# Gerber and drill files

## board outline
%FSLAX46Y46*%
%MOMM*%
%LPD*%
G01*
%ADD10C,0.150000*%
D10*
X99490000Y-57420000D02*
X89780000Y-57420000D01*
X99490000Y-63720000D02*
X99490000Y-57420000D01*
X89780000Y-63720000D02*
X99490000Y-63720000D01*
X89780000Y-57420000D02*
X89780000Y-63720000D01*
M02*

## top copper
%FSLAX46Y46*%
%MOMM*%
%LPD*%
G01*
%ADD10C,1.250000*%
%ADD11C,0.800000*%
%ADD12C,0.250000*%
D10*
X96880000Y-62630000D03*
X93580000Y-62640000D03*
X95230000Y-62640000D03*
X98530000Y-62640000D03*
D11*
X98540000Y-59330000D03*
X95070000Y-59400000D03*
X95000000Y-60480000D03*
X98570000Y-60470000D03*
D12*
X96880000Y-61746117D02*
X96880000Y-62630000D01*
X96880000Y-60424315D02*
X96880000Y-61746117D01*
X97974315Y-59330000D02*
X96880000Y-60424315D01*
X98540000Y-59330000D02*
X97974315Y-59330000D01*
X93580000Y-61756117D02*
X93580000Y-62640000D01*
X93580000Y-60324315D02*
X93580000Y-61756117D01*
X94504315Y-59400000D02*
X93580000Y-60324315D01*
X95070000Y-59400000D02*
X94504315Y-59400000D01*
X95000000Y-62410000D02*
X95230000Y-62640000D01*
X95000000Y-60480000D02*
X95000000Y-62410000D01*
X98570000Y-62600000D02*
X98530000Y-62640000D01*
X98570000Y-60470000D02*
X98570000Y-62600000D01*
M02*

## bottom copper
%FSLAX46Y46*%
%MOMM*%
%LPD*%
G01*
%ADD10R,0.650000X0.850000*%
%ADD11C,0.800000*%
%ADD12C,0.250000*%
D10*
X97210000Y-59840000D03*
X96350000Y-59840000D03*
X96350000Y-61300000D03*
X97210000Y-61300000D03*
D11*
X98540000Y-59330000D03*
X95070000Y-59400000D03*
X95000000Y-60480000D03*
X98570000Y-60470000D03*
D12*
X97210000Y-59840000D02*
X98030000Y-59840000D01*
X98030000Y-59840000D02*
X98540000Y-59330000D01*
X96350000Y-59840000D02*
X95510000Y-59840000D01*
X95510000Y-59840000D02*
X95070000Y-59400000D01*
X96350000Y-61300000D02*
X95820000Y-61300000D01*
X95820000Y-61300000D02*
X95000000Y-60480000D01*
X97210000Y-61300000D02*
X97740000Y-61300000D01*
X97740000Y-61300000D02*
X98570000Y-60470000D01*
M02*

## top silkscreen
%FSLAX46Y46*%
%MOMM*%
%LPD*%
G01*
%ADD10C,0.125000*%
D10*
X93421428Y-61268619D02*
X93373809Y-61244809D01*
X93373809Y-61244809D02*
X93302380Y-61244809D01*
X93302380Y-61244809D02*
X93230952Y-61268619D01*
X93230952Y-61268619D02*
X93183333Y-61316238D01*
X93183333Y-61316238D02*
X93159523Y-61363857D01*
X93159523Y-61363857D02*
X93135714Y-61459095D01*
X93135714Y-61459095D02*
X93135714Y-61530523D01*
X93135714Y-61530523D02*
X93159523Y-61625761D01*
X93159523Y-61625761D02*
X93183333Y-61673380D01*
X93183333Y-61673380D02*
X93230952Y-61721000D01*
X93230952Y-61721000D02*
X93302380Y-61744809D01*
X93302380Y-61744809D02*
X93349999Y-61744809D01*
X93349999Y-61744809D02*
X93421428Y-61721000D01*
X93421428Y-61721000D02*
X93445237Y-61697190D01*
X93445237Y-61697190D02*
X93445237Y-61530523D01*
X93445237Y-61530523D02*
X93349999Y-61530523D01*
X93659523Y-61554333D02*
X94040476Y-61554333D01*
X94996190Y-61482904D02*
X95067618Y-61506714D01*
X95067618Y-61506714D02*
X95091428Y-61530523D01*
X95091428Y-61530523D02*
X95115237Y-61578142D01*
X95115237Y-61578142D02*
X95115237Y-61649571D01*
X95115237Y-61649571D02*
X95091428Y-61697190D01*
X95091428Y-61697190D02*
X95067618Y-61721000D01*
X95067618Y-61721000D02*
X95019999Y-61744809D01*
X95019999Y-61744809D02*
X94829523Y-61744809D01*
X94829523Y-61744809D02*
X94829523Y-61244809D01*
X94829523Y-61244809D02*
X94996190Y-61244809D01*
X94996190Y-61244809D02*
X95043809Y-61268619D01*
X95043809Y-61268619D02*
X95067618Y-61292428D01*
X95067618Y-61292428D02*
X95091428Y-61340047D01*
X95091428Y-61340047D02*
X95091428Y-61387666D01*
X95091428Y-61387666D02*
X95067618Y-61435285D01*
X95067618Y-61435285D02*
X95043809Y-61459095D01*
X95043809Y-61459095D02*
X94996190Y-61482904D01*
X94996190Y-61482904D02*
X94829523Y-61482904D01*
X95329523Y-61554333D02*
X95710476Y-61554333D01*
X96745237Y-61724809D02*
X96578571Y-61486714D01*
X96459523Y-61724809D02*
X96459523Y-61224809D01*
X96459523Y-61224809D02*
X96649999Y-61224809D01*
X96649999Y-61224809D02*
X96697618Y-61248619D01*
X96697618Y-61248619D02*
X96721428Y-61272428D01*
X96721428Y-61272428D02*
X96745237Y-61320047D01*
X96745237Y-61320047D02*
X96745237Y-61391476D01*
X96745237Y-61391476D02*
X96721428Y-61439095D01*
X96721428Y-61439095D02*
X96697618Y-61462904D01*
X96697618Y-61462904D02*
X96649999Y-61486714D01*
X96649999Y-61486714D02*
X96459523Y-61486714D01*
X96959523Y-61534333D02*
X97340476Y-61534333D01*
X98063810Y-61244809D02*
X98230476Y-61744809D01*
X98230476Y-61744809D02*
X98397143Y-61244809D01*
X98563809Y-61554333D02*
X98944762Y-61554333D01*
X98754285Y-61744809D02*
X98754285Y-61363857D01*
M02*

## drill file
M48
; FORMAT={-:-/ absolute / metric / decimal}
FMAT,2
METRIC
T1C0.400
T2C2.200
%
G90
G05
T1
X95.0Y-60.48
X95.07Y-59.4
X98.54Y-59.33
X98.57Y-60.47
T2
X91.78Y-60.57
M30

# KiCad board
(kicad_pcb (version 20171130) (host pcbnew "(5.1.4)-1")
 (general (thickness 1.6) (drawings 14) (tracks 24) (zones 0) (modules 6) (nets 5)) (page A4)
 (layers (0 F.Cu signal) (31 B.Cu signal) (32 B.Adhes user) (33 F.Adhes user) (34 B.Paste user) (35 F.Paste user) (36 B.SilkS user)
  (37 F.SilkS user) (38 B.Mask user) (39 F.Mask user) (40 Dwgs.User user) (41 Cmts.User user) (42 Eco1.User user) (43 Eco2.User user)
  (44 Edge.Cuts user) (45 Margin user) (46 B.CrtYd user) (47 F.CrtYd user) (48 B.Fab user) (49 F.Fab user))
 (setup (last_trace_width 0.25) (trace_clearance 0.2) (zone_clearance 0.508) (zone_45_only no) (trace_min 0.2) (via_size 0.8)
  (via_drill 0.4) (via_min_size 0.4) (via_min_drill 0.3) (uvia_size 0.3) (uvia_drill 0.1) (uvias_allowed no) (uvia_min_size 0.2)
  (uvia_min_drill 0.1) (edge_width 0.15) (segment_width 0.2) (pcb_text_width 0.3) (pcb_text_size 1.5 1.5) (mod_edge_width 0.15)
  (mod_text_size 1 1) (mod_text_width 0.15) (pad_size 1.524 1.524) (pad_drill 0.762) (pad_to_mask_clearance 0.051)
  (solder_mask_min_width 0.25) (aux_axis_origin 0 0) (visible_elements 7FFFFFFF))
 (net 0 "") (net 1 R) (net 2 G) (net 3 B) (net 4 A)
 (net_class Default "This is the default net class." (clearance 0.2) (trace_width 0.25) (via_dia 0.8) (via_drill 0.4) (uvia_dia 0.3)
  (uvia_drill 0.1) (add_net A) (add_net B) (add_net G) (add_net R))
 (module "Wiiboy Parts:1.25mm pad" (layer F.Cu) (at 96.88 62.63)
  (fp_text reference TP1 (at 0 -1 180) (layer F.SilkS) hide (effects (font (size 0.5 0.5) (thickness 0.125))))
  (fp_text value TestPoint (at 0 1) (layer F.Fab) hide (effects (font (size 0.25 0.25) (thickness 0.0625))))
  (pad 1 smd circle (at 0 0) (size 1.25 1.25) (layers F.Cu F.Paste F.Mask) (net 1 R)))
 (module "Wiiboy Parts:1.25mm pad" (layer F.Cu) (at 93.58 62.64)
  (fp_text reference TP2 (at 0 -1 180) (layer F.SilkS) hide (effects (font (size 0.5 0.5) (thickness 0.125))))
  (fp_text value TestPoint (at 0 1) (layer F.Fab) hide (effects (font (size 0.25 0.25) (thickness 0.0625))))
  (pad 1 smd circle (at 0 0) (size 1.25 1.25) (layers F.Cu F.Paste F.Mask) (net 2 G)))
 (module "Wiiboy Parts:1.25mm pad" (layer F.Cu) (at 95.23 62.64)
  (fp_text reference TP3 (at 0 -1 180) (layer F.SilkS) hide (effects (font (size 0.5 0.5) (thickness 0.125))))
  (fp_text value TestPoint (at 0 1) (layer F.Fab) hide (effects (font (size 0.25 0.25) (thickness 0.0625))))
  (pad 1 smd circle (at 0 0) (size 1.25 1.25) (layers F.Cu F.Paste F.Mask) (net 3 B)))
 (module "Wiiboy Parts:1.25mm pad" (layer F.Cu) (at 98.53 62.64)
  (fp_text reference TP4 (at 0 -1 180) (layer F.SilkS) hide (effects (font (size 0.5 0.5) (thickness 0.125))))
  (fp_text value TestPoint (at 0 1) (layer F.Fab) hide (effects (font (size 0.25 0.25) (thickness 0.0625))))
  (pad 1 smd circle (at 0 0) (size 1.25 1.25) (layers F.Cu F.Paste F.Mask) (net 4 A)))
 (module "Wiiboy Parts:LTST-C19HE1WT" (layer B.Cu) (at 96.78 60.57 180)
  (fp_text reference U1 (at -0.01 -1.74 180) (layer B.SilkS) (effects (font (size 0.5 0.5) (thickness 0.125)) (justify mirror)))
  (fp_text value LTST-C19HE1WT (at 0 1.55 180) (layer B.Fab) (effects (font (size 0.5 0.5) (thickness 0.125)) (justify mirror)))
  (pad 1 smd rect (at -0.43 0.73 180) (size 0.65 0.85) (layers B.Cu B.Paste B.Mask) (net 1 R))
  (pad 2 smd rect (at 0.43 0.73 180) (size 0.65 0.85) (layers B.Cu B.Paste B.Mask) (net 2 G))
  (pad 3 smd rect (at 0.43 -0.73 180) (size 0.65 0.85) (layers B.Cu B.Paste B.Mask) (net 3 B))
  (pad 4 smd rect (at -0.43 -0.73 180) (size 0.65 0.85) (layers B.Cu B.Paste B.Mask) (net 4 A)))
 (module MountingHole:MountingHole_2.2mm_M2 (layer F.Cu) (at 91.78 60.57)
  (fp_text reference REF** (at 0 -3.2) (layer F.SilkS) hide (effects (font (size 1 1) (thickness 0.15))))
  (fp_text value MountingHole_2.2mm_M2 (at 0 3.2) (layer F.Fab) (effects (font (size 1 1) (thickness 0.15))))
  (pad 1 np_thru_hole circle (at 0 0) (size 2.2 2.2) (drill 2.2) (layers *.Cu *.Mask)))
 (gr_line (start 99.49 57.42) (end 89.78 57.42) (layer Edge.Cuts) (width 0.15))
 (gr_line (start 99.49 63.72) (end 99.49 57.42) (layer Edge.Cuts) (width 0.15))
 (gr_line (start 89.78 63.72) (end 99.49 63.72) (layer Edge.Cuts) (width 0.15))
 (gr_line (start 89.78 57.42) (end 89.78 63.72) (layer Edge.Cuts) (width 0.15))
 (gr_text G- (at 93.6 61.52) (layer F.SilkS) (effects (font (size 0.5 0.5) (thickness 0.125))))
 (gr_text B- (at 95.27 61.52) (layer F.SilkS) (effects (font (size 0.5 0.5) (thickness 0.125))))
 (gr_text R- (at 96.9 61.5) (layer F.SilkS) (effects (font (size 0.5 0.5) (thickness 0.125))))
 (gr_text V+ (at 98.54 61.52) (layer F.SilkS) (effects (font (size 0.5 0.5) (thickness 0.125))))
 (via (at 98.54 59.33) (size 0.8) (drill 0.4) (layers F.Cu B.Cu) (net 1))
 (segment (start 97.21 59.84) (end 98.03 59.84) (width 0.25) (layer B.Cu) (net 1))
 (segment (start 98.03 59.84) (end 98.54 59.33) (width 0.25) (layer B.Cu) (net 1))
 (segment (start 96.88 61.746117) (end 96.88 62.63) (width 0.25) (layer F.Cu) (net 1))
 (segment (start 96.88 60.424315) (end 96.88 61.746117) (width 0.25) (layer F.Cu) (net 1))
 (segment (start 97.974315 59.33) (end 96.88 60.424315) (width 0.25) (layer F.Cu) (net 1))
 (segment (start 98.54 59.33) (end 97.974315 59.33) (width 0.25) (layer F.Cu) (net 1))
 (via (at 95.07 59.4) (size 0.8) (drill 0.4) (layers F.Cu B.Cu) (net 2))
 (segment (start 96.35 59.84) (end 95.51 59.84) (width 0.25) (layer B.Cu) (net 2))
 (segment (start 95.51 59.84) (end 95.07 59.4) (width 0.25) (layer B.Cu) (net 2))
 (segment (start 93.58 61.756117) (end 93.58 62.64) (width 0.25) (layer F.Cu) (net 2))
 (segment (start 93.58 60.324315) (end 93.58 61.756117) (width 0.25) (layer F.Cu) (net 2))
 (segment (start 94.504315 59.4) (end 93.58 60.324315) (width 0.25) (layer F.Cu) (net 2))
 (segment (start 95.07 59.4) (end 94.504315 59.4) (width 0.25) (layer F.Cu) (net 2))
 (via (at 95 60.48) (size 0.8) (drill 0.4) (layers F.Cu B.Cu) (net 3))
 (segment (start 96.35 61.3) (end 95.82 61.3) (width 0.25) (layer B.Cu) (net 3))
 (segment (start 95.82 61.3) (end 95 60.48) (width 0.25) (layer B.Cu) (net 3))
 (segment (start 95 62.41) (end 95.23 62.64) (width 0.25) (layer F.Cu) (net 3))
 (segment (start 95 60.48) (end 95 62.41) (width 0.25) (layer F.Cu) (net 3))
 (via (at 98.57 60.47) (size 0.8) (drill 0.4) (layers F.Cu B.Cu) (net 4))
 (segment (start 97.21 61.3) (end 97.74 61.3) (width 0.25) (layer B.Cu) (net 4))
 (segment (start 97.74 61.3) (end 98.57 60.47) (width 0.25) (layer B.Cu) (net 4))
 (segment (start 98.57 62.6) (end 98.53 62.64) (width 0.25) (layer F.Cu) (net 4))
 (segment (start 98.57 60.47) (end 98.57 62.6) (width 0.25) (layer F.Cu) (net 4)))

